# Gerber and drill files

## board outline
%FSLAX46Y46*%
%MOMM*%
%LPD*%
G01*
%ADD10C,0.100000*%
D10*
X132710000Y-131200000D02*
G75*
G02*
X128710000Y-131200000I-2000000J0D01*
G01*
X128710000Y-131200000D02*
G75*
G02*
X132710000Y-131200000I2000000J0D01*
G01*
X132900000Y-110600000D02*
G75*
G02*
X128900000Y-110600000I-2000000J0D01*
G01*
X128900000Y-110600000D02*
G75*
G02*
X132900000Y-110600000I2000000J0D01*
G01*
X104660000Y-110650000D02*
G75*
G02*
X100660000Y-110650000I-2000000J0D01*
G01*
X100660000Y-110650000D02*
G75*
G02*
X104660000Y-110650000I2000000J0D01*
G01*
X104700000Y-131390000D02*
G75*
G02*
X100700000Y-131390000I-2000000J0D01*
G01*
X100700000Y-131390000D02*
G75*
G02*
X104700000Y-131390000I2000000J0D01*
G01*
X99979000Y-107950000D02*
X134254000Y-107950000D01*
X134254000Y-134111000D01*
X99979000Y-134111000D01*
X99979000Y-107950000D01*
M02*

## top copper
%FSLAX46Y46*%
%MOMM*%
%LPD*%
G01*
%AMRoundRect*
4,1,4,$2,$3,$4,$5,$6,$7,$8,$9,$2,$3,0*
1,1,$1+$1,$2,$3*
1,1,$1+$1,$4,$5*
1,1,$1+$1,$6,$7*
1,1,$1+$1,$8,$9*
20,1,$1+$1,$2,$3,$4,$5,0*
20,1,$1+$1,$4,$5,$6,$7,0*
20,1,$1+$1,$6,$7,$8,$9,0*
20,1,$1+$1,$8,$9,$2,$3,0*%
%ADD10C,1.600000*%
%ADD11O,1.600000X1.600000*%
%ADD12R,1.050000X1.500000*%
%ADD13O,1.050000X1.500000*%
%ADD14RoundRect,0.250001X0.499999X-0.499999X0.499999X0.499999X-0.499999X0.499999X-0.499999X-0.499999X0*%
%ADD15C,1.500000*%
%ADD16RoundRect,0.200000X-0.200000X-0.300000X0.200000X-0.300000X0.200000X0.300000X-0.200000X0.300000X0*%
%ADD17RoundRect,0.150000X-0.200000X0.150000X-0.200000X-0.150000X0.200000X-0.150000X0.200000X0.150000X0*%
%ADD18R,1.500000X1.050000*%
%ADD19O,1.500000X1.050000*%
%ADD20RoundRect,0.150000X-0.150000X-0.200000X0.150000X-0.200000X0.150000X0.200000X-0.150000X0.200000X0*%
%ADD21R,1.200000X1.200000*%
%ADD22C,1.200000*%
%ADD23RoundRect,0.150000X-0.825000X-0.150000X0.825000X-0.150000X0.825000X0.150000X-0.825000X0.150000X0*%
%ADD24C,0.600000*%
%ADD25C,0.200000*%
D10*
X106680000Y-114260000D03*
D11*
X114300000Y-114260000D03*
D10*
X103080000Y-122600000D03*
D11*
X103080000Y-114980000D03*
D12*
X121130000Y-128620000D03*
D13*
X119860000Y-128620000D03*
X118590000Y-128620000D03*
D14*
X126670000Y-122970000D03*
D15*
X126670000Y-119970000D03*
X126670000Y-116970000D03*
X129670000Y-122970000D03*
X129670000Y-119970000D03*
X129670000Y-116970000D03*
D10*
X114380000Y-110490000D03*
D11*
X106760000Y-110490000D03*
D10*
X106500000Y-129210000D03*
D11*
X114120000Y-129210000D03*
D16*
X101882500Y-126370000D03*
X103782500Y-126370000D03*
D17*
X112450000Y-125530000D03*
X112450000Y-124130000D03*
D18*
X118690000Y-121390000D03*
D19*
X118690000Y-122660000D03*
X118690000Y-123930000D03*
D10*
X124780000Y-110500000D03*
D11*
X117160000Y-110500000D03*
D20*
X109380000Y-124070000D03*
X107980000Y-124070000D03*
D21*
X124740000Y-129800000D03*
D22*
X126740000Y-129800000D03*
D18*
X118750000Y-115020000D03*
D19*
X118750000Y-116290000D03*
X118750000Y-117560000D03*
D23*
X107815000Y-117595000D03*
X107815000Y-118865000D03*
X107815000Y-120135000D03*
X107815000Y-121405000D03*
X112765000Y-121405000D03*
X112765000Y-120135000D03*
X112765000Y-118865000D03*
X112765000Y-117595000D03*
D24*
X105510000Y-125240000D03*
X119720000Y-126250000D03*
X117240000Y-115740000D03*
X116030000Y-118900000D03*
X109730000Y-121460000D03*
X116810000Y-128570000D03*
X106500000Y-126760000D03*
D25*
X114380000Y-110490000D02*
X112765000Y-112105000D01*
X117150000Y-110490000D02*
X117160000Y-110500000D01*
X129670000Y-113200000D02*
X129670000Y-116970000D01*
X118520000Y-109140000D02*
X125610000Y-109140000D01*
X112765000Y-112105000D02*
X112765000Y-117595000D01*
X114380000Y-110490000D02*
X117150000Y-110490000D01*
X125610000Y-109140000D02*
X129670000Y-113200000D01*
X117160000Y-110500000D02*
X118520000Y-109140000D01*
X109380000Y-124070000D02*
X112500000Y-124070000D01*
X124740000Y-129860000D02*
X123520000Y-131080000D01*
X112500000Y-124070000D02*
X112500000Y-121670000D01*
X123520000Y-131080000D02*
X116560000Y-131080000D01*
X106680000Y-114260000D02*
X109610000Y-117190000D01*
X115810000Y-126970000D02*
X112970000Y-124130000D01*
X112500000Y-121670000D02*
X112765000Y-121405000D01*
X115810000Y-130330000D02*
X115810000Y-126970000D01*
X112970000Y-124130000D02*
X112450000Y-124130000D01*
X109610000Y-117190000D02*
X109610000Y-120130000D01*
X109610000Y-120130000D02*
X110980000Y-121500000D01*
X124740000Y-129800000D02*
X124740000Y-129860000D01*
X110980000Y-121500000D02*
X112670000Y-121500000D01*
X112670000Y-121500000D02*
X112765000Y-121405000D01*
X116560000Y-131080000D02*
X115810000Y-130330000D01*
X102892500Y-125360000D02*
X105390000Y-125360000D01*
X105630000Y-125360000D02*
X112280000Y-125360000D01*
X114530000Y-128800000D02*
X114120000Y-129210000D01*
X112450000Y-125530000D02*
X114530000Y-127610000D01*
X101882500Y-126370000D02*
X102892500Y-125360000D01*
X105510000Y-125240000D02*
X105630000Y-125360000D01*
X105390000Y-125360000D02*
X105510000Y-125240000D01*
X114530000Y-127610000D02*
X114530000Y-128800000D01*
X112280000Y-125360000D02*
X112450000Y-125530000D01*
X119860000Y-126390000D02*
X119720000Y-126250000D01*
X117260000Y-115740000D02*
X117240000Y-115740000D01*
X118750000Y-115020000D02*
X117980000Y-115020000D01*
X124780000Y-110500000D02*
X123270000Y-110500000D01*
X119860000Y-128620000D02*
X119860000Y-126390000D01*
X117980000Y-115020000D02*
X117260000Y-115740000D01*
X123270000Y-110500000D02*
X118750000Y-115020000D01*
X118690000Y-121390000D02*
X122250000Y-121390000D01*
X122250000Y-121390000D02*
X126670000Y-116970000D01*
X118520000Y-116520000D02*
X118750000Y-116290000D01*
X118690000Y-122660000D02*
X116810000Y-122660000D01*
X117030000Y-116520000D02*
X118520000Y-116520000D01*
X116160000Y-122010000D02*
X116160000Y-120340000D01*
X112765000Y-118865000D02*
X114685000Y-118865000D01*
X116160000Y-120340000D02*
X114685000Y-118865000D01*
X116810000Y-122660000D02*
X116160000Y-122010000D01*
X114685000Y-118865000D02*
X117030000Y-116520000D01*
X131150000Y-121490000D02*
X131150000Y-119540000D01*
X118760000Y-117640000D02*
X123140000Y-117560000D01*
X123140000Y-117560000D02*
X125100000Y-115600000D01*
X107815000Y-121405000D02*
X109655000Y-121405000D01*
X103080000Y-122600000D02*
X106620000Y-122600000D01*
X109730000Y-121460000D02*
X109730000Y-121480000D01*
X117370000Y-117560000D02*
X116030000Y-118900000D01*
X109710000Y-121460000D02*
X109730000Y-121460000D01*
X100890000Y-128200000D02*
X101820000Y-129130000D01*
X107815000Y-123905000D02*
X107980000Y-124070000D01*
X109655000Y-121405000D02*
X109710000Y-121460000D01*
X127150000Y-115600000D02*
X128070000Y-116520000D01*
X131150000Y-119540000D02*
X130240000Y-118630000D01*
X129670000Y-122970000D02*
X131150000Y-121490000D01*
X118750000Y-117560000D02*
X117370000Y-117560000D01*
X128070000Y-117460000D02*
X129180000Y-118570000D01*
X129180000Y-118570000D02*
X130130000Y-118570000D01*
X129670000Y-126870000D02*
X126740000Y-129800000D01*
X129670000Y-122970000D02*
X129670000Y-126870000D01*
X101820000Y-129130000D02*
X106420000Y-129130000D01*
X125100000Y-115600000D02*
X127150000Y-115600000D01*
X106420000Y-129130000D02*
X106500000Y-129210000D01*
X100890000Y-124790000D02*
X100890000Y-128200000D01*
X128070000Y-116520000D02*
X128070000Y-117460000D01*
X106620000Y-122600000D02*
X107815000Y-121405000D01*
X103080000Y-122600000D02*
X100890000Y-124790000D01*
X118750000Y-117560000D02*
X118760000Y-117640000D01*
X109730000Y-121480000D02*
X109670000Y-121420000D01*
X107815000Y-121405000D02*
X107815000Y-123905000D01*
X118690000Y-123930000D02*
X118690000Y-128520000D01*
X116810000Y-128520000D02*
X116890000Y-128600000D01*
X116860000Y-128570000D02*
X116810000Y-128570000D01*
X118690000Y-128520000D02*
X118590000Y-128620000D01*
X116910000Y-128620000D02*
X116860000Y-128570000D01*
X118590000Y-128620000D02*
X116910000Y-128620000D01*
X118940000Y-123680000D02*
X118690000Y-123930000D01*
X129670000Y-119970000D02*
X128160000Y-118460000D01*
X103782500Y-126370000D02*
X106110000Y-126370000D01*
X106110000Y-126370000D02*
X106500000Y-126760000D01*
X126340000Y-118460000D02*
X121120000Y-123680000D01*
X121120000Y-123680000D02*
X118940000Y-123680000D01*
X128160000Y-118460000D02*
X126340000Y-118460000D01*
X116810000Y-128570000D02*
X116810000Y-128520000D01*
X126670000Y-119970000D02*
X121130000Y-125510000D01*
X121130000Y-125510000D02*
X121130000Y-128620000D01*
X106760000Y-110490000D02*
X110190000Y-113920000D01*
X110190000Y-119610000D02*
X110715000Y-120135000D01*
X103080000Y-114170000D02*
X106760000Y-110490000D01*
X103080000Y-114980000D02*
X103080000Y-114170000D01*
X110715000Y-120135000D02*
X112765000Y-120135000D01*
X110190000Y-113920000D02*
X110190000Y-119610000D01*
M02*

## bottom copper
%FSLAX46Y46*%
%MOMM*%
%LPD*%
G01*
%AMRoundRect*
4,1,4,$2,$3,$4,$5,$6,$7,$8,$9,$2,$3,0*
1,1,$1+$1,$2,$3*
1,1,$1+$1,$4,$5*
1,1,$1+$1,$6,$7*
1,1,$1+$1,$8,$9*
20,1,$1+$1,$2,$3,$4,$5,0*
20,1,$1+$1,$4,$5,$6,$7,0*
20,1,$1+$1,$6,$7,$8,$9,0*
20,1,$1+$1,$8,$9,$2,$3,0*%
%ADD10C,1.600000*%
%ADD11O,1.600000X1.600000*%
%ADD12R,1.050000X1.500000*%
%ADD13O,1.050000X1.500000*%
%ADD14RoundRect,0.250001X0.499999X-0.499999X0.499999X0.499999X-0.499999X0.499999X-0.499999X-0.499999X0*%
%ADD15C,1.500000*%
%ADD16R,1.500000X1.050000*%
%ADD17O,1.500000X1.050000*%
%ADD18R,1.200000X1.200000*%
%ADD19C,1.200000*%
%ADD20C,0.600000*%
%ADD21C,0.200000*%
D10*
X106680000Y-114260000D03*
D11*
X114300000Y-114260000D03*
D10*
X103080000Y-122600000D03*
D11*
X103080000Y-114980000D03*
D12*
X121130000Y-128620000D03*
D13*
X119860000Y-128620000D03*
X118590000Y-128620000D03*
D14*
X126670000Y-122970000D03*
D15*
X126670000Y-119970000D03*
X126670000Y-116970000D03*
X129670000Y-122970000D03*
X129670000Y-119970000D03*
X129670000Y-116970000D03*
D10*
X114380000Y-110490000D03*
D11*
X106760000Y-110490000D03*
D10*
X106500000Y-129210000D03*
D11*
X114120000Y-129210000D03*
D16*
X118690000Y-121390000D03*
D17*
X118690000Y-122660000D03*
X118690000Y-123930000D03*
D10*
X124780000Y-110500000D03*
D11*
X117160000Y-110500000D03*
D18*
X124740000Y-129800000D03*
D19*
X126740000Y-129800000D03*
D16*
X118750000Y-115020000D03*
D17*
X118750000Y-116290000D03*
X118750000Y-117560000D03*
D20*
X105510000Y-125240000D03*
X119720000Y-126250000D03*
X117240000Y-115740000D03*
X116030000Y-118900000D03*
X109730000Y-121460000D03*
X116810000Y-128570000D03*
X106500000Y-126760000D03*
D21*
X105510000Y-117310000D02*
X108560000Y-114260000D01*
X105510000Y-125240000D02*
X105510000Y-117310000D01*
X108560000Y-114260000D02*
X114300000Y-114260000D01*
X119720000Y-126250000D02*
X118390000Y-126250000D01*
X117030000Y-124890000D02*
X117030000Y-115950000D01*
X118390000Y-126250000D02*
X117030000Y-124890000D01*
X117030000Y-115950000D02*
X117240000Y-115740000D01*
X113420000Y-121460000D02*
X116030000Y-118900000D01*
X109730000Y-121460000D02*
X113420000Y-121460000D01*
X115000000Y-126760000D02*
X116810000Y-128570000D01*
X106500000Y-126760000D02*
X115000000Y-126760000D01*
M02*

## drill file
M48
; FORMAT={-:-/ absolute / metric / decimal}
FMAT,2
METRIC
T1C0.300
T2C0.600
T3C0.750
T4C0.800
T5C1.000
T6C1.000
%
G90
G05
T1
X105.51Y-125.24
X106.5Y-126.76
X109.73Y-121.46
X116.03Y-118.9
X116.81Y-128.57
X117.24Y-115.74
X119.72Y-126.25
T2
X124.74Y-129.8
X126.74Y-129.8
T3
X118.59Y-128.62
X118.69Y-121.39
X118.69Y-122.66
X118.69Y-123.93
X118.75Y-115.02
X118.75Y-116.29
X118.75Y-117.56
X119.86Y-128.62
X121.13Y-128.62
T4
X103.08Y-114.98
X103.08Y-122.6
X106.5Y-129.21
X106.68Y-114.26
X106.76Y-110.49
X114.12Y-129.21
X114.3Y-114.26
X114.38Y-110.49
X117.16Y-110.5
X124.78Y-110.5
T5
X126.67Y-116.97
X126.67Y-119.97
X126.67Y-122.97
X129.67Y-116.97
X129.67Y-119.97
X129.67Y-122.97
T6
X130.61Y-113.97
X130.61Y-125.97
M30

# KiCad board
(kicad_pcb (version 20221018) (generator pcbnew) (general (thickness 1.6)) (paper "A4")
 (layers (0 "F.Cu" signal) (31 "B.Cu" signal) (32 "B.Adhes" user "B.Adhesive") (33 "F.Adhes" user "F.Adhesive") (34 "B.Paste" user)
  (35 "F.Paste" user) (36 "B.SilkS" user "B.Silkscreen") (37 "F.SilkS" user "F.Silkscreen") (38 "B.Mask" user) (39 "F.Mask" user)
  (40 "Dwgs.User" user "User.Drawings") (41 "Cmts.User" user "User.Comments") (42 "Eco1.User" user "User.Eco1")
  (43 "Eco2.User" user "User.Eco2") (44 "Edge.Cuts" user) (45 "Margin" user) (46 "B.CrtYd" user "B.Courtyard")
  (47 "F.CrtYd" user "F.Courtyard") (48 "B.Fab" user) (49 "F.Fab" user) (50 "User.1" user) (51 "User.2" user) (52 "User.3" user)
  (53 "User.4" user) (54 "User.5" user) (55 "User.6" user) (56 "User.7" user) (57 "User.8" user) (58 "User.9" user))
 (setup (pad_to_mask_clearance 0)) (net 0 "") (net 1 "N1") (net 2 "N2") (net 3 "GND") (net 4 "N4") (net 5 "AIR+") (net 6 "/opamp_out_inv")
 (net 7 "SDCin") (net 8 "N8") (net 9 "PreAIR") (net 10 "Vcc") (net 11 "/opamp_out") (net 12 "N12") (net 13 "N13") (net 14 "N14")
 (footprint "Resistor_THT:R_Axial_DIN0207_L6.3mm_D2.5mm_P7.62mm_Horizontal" (layer "F.Cu") (at 106.68 114.26)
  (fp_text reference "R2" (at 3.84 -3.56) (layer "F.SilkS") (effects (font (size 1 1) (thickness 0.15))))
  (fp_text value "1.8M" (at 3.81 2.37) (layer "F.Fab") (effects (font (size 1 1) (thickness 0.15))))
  (pad "1" thru_hole circle (at 0 0) (size 1.6 1.6) (drill 0.8) (layers "*.Cu" "*.Mask") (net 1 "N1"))
  (pad "2" thru_hole oval (at 7.62 0) (size 1.6 1.6) (drill 0.8) (layers "*.Cu" "*.Mask") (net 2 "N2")))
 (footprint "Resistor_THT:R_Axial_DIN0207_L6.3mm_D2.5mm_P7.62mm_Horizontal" (layer "F.Cu") (at 103.08 122.6 90)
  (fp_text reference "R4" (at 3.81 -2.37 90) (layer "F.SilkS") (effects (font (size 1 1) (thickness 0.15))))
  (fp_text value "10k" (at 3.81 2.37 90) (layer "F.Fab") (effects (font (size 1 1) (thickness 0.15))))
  (pad "1" thru_hole circle (at 0 0 90) (size 1.6 1.6) (drill 0.8) (layers "*.Cu" "*.Mask") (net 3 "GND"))
  (pad "2" thru_hole oval (at 7.62 0 90) (size 1.6 1.6) (drill 0.8) (layers "*.Cu" "*.Mask") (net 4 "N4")))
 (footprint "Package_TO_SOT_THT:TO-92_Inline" (layer "F.Cu") (at 121.13 128.62 180)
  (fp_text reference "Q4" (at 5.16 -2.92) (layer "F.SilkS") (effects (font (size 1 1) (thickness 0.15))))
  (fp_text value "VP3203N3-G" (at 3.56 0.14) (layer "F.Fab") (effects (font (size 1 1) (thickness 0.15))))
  (pad "1" thru_hole rect (at 0 0 180) (size 1.05 1.5) (drill 0.75) (layers "*.Cu" "*.Mask") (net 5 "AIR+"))
  (pad "2" thru_hole oval (at 1.27 0 180) (size 1.05 1.5) (drill 0.75) (layers "*.Cu" "*.Mask") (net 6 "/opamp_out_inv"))
  (pad "3" thru_hole oval (at 2.54 0 180) (size 1.05 1.5) (drill 0.75) (layers "*.Cu" "*.Mask") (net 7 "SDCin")))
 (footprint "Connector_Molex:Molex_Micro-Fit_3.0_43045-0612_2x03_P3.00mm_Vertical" (layer "F.Cu") (at 126.67 122.97 90)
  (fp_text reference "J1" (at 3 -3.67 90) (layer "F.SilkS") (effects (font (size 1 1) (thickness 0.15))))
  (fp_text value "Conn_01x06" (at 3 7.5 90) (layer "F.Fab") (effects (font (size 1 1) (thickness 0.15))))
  (pad "" np_thru_hole circle (at -3 3.94 90) (size 1 1) (drill 1) (layers "*.Cu" "*.Mask"))
  (pad "" np_thru_hole circle (at 9 3.94 90) (size 1 1) (drill 1) (layers "*.Cu" "*.Mask"))
  (pad "1" thru_hole roundrect (at 0 0 90) (size 1.5 1.5) (drill 1) (layers "*.Cu" "*.Mask") (roundrect_rratio 0.166667) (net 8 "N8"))
  (pad "2" thru_hole circle (at 3 0 90) (size 1.5 1.5) (drill 1) (layers "*.Cu" "*.Mask") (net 5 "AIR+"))
  (pad "3" thru_hole circle (at 6 0 90) (size 1.5 1.5) (drill 1) (layers "*.Cu" "*.Mask") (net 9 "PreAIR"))
  (pad "4" thru_hole circle (at 0 3 90) (size 1.5 1.5) (drill 1) (layers "*.Cu" "*.Mask") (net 3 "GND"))
  (pad "5" thru_hole circle (at 3 3 90) (size 1.5 1.5) (drill 1) (layers "*.Cu" "*.Mask") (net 7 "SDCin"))
  (pad "6" thru_hole circle (at 6 3 90) (size 1.5 1.5) (drill 1) (layers "*.Cu" "*.Mask") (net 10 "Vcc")))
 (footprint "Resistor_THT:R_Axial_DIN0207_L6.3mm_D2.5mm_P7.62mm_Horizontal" (layer "F.Cu") (at 114.38 110.49 180)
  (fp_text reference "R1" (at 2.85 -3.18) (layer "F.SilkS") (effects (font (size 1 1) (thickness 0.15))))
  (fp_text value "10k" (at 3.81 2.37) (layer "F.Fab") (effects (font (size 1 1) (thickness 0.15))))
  (pad "1" thru_hole circle (at 0 0 180) (size 1.6 1.6) (drill 0.8) (layers "*.Cu" "*.Mask") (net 10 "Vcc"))
  (pad "2" thru_hole oval (at 7.62 0 180) (size 1.6 1.6) (drill 0.8) (layers "*.Cu" "*.Mask") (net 4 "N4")))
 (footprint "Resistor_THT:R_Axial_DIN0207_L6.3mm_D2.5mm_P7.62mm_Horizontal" (layer "F.Cu") (at 106.5 129.21)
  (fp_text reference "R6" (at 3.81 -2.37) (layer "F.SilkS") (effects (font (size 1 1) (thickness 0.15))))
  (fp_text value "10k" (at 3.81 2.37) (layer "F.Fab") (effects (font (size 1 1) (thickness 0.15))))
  (pad "1" thru_hole circle (at 0 0) (size 1.6 1.6) (drill 0.8) (layers "*.Cu" "*.Mask") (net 3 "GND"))
  (pad "2" thru_hole oval (at 7.62 0) (size 1.6 1.6) (drill 0.8) (layers "*.Cu" "*.Mask") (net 2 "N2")))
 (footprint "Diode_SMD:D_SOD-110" (layer "F.Cu") (at 102.8325 126.37)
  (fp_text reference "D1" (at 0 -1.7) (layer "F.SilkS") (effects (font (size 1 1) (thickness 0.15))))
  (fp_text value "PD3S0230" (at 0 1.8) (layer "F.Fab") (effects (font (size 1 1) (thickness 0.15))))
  (pad "1" smd roundrect (at -0.95 0) (size 0.8 1) (layers "F.Cu" "F.Paste" "F.Mask") (roundrect_rratio 0.25) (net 2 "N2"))
  (pad "2" smd roundrect (at 0.95 0) (size 0.8 1) (layers "F.Cu" "F.Paste" "F.Mask") (roundrect_rratio 0.25) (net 7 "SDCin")))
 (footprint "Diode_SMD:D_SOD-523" (layer "F.Cu") (at 112.45 124.83 90)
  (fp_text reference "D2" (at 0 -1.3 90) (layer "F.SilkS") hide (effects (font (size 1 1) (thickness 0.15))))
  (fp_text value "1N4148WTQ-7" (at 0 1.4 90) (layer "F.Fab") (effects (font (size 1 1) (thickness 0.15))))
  (pad "1" smd roundrect (at -0.7 0 270) (size 0.6 0.7) (layers "F.Cu" "F.Paste" "F.Mask") (roundrect_rratio 0.25) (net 2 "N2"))
  (pad "2" smd roundrect (at 0.7 0 270) (size 0.6 0.7) (layers "F.Cu" "F.Paste" "F.Mask") (roundrect_rratio 0.25) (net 1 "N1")))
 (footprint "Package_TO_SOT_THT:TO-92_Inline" (layer "F.Cu") (at 118.69 121.39 -90)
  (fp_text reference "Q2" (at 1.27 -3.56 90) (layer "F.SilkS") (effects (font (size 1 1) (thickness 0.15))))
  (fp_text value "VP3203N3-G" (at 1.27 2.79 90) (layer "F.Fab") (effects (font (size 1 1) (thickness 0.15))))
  (pad "1" thru_hole rect (at 0 0 270) (size 1.05 1.5) (drill 0.75) (layers "*.Cu" "*.Mask") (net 9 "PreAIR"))
  (pad "2" thru_hole oval (at 1.27 0 270) (size 1.05 1.5) (drill 0.75) (layers "*.Cu" "*.Mask") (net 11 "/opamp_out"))
  (pad "3" thru_hole oval (at 2.54 0 270) (size 1.05 1.5) (drill 0.75) (layers "*.Cu" "*.Mask") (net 7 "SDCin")))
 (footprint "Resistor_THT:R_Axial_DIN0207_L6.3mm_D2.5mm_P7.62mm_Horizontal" (layer "F.Cu") (at 124.78 110.5 180)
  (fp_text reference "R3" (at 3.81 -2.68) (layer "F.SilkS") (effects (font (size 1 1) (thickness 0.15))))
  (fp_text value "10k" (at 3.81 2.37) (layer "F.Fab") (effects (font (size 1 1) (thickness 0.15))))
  (pad "1" thru_hole circle (at 0 0 180) (size 1.6 1.6) (drill 0.8) (layers "*.Cu" "*.Mask") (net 6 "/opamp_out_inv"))
  (pad "2" thru_hole oval (at 7.62 0 180) (size 1.6 1.6) (drill 0.8) (layers "*.Cu" "*.Mask") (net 10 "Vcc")))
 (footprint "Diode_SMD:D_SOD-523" (layer "F.Cu") (at 108.68 124.07 180)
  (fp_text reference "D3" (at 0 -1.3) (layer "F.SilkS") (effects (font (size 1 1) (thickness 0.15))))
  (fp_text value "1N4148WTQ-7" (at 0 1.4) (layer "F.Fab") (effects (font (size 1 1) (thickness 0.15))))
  (pad "1" smd roundrect (at -0.7 0) (size 0.6 0.7) (layers "F.Cu" "F.Paste" "F.Mask") (roundrect_rratio 0.25) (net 1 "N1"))
  (pad "2" smd roundrect (at 0.7 0) (size 0.6 0.7) (layers "F.Cu" "F.Paste" "F.Mask") (roundrect_rratio 0.25) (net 3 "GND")))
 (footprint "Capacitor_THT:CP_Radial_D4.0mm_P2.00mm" (layer "F.Cu") (at 124.74 129.8)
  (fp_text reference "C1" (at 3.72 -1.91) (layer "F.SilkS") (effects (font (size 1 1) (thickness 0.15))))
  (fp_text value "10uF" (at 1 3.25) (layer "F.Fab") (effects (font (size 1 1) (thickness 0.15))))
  (pad "1" thru_hole rect (at 0 0) (size 1.2 1.2) (drill 0.6) (layers "*.Cu" "*.Mask") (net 1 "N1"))
  (pad "2" thru_hole circle (at 2 0) (size 1.2 1.2) (drill 0.6) (layers "*.Cu" "*.Mask") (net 3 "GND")))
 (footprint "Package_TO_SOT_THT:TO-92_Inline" (layer "F.Cu") (at 118.75 115.02 -90)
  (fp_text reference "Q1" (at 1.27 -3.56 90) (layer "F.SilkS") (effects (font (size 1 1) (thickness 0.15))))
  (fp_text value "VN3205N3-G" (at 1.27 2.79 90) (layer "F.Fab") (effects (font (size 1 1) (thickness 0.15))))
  (pad "1" thru_hole rect (at 0 0 270) (size 1.05 1.5) (drill 0.75) (layers "*.Cu" "*.Mask") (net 6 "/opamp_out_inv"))
  (pad "2" thru_hole oval (at 1.27 0 270) (size 1.05 1.5) (drill 0.75) (layers "*.Cu" "*.Mask") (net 11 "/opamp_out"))
  (pad "3" thru_hole oval (at 2.54 0 270) (size 1.05 1.5) (drill 0.75) (layers "*.Cu" "*.Mask") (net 3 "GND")))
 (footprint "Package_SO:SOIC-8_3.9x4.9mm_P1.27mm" (layer "F.Cu") (at 110.29 119.5)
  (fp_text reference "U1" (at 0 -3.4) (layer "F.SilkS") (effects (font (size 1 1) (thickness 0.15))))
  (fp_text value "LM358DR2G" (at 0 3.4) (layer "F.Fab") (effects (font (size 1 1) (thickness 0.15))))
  (pad "1" smd roundrect (at -2.475 -1.905) (size 1.95 0.6) (layers "F.Cu" "F.Paste" "F.Mask") (roundrect_rratio 0.25) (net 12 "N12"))
  (pad "2" smd roundrect (at -2.475 -0.635) (size 1.95 0.6) (layers "F.Cu" "F.Paste" "F.Mask") (roundrect_rratio 0.25) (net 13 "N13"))
  (pad "3" smd roundrect (at -2.475 0.635) (size 1.95 0.6) (layers "F.Cu" "F.Paste" "F.Mask") (roundrect_rratio 0.25) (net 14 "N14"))
  (pad "4" smd roundrect (at -2.475 1.905) (size 1.95 0.6) (layers "F.Cu" "F.Paste" "F.Mask") (roundrect_rratio 0.25) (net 3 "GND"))
  (pad "5" smd roundrect (at 2.475 1.905) (size 1.95 0.6) (layers "F.Cu" "F.Paste" "F.Mask") (roundrect_rratio 0.25) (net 1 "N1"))
  (pad "6" smd roundrect (at 2.475 0.635) (size 1.95 0.6) (layers "F.Cu" "F.Paste" "F.Mask") (roundrect_rratio 0.25) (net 4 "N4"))
  (pad "7" smd roundrect (at 2.475 -0.635) (size 1.95 0.6) (layers "F.Cu" "F.Paste" "F.Mask") (roundrect_rratio 0.25) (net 11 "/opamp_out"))
  (pad "8" smd roundrect (at 2.475 -1.905) (size 1.95 0.6) (layers "F.Cu" "F.Paste" "F.Mask") (roundrect_rratio 0.25) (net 10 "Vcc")))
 (gr_circle (center 130.71 131.2) (end 132.71 131.2) (stroke (width 0.1) (type default)) (fill none) (layer "Edge.Cuts"))
 (gr_circle (center 130.9 110.6) (end 132.9 110.6) (stroke (width 0.1) (type default)) (fill none) (layer "Edge.Cuts"))
 (gr_circle (center 102.66 110.65) (end 104.66 110.65) (stroke (width 0.1) (type default)) (fill none) (layer "Edge.Cuts"))
 (gr_circle (center 102.7 131.39) (end 104.7 131.39) (stroke (width 0.1) (type default)) (fill none) (layer "Edge.Cuts"))
 (gr_rect (start 99.979 107.95) (end 134.254 134.111) (stroke (width 0.1) (type solid)) (fill none) (layer "Edge.Cuts"))
 (segment (start 114.38 110.49) (end 112.765 112.105) (width 0.2) (layer "F.Cu") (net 10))
 (segment (start 117.15 110.49) (end 117.16 110.5) (width 0.2) (layer "F.Cu") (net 10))
 (segment (start 129.67 113.2) (end 129.67 116.97) (width 0.2) (layer "F.Cu") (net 10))
 (segment (start 118.52 109.14) (end 125.61 109.14) (width 0.2) (layer "F.Cu") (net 10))
 (segment (start 112.765 112.105) (end 112.765 117.595) (width 0.2) (layer "F.Cu") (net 10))
 (segment (start 114.38 110.49) (end 117.15 110.49) (width 0.2) (layer "F.Cu") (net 10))
 (segment (start 125.61 109.14) (end 129.67 113.2) (width 0.2) (layer "F.Cu") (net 10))
 (segment (start 117.16 110.5) (end 118.52 109.14) (width 0.2) (layer "F.Cu") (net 10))
 (segment (start 109.38 124.07) (end 112.5 124.07) (width 0.2) (layer "F.Cu") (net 1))
 (segment (start 124.74 129.86) (end 123.52 131.08) (width 0.2) (layer "F.Cu") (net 1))
 (segment (start 112.5 124.07) (end 112.5 121.67) (width 0.2) (layer "F.Cu") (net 1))
 (segment (start 123.52 131.08) (end 116.56 131.08) (width 0.2) (layer "F.Cu") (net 1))
 (segment (start 106.68 114.26) (end 109.61 117.19) (width 0.2) (layer "F.Cu") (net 1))
 (segment (start 115.81 126.97) (end 112.97 124.13) (width 0.2) (layer "F.Cu") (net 1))
 (segment (start 112.5 121.67) (end 112.765 121.405) (width 0.2) (layer "F.Cu") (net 1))
 (segment (start 115.81 130.33) (end 115.81 126.97) (width 0.2) (layer "F.Cu") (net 1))
 (segment (start 112.97 124.13) (end 112.45 124.13) (width 0.2) (layer "F.Cu") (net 1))
 (segment (start 109.61 117.19) (end 109.61 120.13) (width 0.2) (layer "F.Cu") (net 1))
 (segment (start 109.61 120.13) (end 110.98 121.5) (width 0.2) (layer "F.Cu") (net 1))
 (segment (start 124.74 129.8) (end 124.74 129.86) (width 0.2) (layer "F.Cu") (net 1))
 (segment (start 110.98 121.5) (end 112.67 121.5) (width 0.2) (layer "F.Cu") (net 1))
 (segment (start 112.67 121.5) (end 112.765 121.405) (width 0.2) (layer "F.Cu") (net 1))
 (segment (start 116.56 131.08) (end 115.81 130.33) (width 0.2) (layer "F.Cu") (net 1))
 (segment (start 102.8925 125.36) (end 105.39 125.36) (width 0.2) (layer "F.Cu") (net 2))
 (segment (start 105.63 125.36) (end 112.28 125.36) (width 0.2) (layer "F.Cu") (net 2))
 (segment (start 114.53 128.8) (end 114.12 129.21) (width 0.2) (layer "F.Cu") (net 2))
 (segment (start 112.45 125.53) (end 114.53 127.61) (width 0.2) (layer "F.Cu") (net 2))
 (segment (start 101.8825 126.37) (end 102.8925 125.36) (width 0.2) (layer "F.Cu") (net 2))
 (segment (start 105.51 125.24) (end 105.63 125.36) (width 0.2) (layer "F.Cu") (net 2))
 (segment (start 105.39 125.36) (end 105.51 125.24) (width 0.2) (layer "F.Cu") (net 2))
 (segment (start 114.53 127.61) (end 114.53 128.8) (width 0.2) (layer "F.Cu") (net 2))
 (segment (start 112.28 125.36) (end 112.45 125.53) (width 0.2) (layer "F.Cu") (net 2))
 (via (at 105.51 125.24) (size 0.6) (drill 0.3) (layers "F.Cu" "B.Cu") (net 2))
 (segment (start 105.51 117.31) (end 108.56 114.26) (width 0.2) (layer "B.Cu") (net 2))
 (segment (start 105.51 125.24) (end 105.51 117.31) (width 0.2) (layer "B.Cu") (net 2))
 (segment (start 108.56 114.26) (end 114.3 114.26) (width 0.2) (layer "B.Cu") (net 2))
 (segment (start 119.86 126.39) (end 119.72 126.25) (width 0.2) (layer "F.Cu") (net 6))
 (segment (start 117.26 115.74) (end 117.24 115.74) (width 0.2) (layer "F.Cu") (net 6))
 (segment (start 118.75 115.02) (end 117.98 115.02) (width 0.2) (layer "F.Cu") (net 6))
 (segment (start 124.78 110.5) (end 123.27 110.5) (width 0.2) (layer "F.Cu") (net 6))
 (segment (start 119.86 128.62) (end 119.86 126.39) (width 0.2) (layer "F.Cu") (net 6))
 (segment (start 117.98 115.02) (end 117.26 115.74) (width 0.2) (layer "F.Cu") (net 6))
 (segment (start 123.27 110.5) (end 118.75 115.02) (width 0.2) (layer "F.Cu") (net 6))
 (via (at 119.72 126.25) (size 0.6) (drill 0.3) (layers "F.Cu" "B.Cu") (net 6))
 (via (at 117.24 115.74) (size 0.6) (drill 0.3) (layers "F.Cu" "B.Cu") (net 6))
 (segment (start 119.72 126.25) (end 118.39 126.25) (width 0.2) (layer "B.Cu") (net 6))
 (segment (start 117.03 124.89) (end 117.03 115.95) (width 0.2) (layer "B.Cu") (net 6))
 (segment (start 118.39 126.25) (end 117.03 124.89) (width 0.2) (layer "B.Cu") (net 6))
 (segment (start 117.03 115.95) (end 117.24 115.74) (width 0.2) (layer "B.Cu") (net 6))
 (segment (start 118.69 121.39) (end 122.25 121.39) (width 0.2) (layer "F.Cu") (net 9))
 (segment (start 122.25 121.39) (end 126.67 116.97) (width 0.2) (layer "F.Cu") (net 9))
 (segment (start 118.52 116.52) (end 118.75 116.29) (width 0.2) (layer "F.Cu") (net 11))
 (segment (start 118.69 122.66) (end 116.81 122.66) (width 0.2) (layer "F.Cu") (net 11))
 (segment (start 117.03 116.52) (end 118.52 116.52) (width 0.2) (layer "F.Cu") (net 11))
 (segment (start 116.16 122.01) (end 116.16 120.34) (width 0.2) (layer "F.Cu") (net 11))
 (segment (start 112.765 118.865) (end 114.685 118.865) (width 0.2) (layer "F.Cu") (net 11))
 (segment (start 116.16 120.34) (end 114.685 118.865) (width 0.2) (layer "F.Cu") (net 11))
 (segment (start 116.81 122.66) (end 116.16 122.01) (width 0.2) (layer "F.Cu") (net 11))
 (segment (start 114.685 118.865) (end 117.03 116.52) (width 0.2) (layer "F.Cu") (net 11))
 (segment (start 131.15 121.49) (end 131.15 119.54) (width 0.2) (layer "F.Cu") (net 3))
 (segment (start 118.76 117.64) (end 123.14 117.56) (width 0.2) (layer "F.Cu") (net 3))
 (segment (start 123.14 117.56) (end 125.1 115.6) (width 0.2) (layer "F.Cu") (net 3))
 (segment (start 107.815 121.405) (end 109.655 121.405) (width 0.2) (layer "F.Cu") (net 3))
 (segment (start 103.08 122.6) (end 106.62 122.6) (width 0.2) (layer "F.Cu") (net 3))
 (segment (start 109.73 121.46) (end 109.73 121.48) (width 0.2) (layer "F.Cu") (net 3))
 (segment (start 117.37 117.56) (end 116.03 118.9) (width 0.2) (layer "F.Cu") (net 3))
 (segment (start 109.71 121.46) (end 109.73 121.46) (width 0.2) (layer "F.Cu") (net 3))
 (segment (start 100.89 128.2) (end 101.82 129.13) (width 0.2) (layer "F.Cu") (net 3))
 (segment (start 107.815 123.905) (end 107.98 124.07) (width 0.2) (layer "F.Cu") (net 3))
 (segment (start 109.655 121.405) (end 109.71 121.46) (width 0.2) (layer "F.Cu") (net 3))
 (segment (start 127.15 115.6) (end 128.07 116.52) (width 0.2) (layer "F.Cu") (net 3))
 (segment (start 131.15 119.54) (end 130.24 118.63) (width 0.2) (layer "F.Cu") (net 3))
 (segment (start 129.67 122.97) (end 131.15 121.49) (width 0.2) (layer "F.Cu") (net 3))
 (segment (start 118.75 117.56) (end 117.37 117.56) (width 0.2) (layer "F.Cu") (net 3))
 (segment (start 128.07 117.46) (end 129.18 118.57) (width 0.2) (layer "F.Cu") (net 3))
 (segment (start 129.18 118.57) (end 130.13 118.57) (width 0.2) (layer "F.Cu") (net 3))
 (segment (start 129.67 126.87) (end 126.74 129.8) (width 0.2) (layer "F.Cu") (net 3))
 (segment (start 129.67 122.97) (end 129.67 126.87) (width 0.2) (layer "F.Cu") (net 3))
 (segment (start 101.82 129.13) (end 106.42 129.13) (width 0.2) (layer "F.Cu") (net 3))
 (segment (start 125.1 115.6) (end 127.15 115.6) (width 0.2) (layer "F.Cu") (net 3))
 (segment (start 106.42 129.13) (end 106.5 129.21) (width 0.2) (layer "F.Cu") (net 3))
 (segment (start 100.89 124.79) (end 100.89 128.2) (width 0.2) (layer "F.Cu") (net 3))
 (segment (start 128.07 116.52) (end 128.07 117.46) (width 0.2) (layer "F.Cu") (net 3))
 (segment (start 106.62 122.6) (end 107.815 121.405) (width 0.2) (layer "F.Cu") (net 3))
 (segment (start 103.08 122.6) (end 100.89 124.79) (width 0.2) (layer "F.Cu") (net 3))
 (segment (start 118.75 117.56) (end 118.76 117.64) (width 0.2) (layer "F.Cu") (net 3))
 (segment (start 109.73 121.48) (end 109.67 121.42) (width 0.2) (layer "F.Cu") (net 3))
 (segment (start 107.815 121.405) (end 107.815 123.905) (width 0.2) (layer "F.Cu") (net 3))
 (via (at 116.03 118.9) (size 0.6) (drill 0.3) (layers "F.Cu" "B.Cu") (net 3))
 (via (at 109.73 121.46) (size 0.6) (drill 0.3) (layers "F.Cu" "B.Cu") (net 3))
 (segment (start 113.42 121.46) (end 116.03 118.9) (width 0.2) (layer "B.Cu") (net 3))
 (segment (start 109.73 121.46) (end 113.42 121.46) (width 0.2) (layer "B.Cu") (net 3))
 (segment (start 118.69 123.93) (end 118.69 128.52) (width 0.2) (layer "F.Cu") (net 7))
 (segment (start 116.81 128.52) (end 116.89 128.6) (width 0.2) (layer "F.Cu") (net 7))
 (segment (start 116.86 128.57) (end 116.81 128.57) (width 0.2) (layer "F.Cu") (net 7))
 (segment (start 118.69 128.52) (end 118.59 128.62) (width 0.2) (layer "F.Cu") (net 7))
 (segment (start 116.91 128.62) (end 116.86 128.57) (width 0.2) (layer "F.Cu") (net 7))
 (segment (start 118.59 128.62) (end 116.91 128.62) (width 0.2) (layer "F.Cu") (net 7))
 (segment (start 118.94 123.68) (end 118.69 123.93) (width 0.2) (layer "F.Cu") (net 7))
 (segment (start 129.67 119.97) (end 128.16 118.46) (width 0.2) (layer "F.Cu") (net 7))
 (segment (start 103.7825 126.37) (end 106.11 126.37) (width 0.2) (layer "F.Cu") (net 7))
 (segment (start 106.11 126.37) (end 106.5 126.76) (width 0.2) (layer "F.Cu") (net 7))
 (segment (start 126.34 118.46) (end 121.12 123.68) (width 0.2) (layer "F.Cu") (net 7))
 (segment (start 121.12 123.68) (end 118.94 123.68) (width 0.2) (layer "F.Cu") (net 7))
 (segment (start 128.16 118.46) (end 126.34 118.46) (width 0.2) (layer "F.Cu") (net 7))
 (segment (start 116.81 128.57) (end 116.81 128.52) (width 0.2) (layer "F.Cu") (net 7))
 (via (at 116.81 128.57) (size 0.6) (drill 0.3) (layers "F.Cu" "B.Cu") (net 7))
 (via (at 106.5 126.76) (size 0.6) (drill 0.3) (layers "F.Cu" "B.Cu") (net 7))
 (segment (start 115 126.76) (end 116.81 128.57) (width 0.2) (layer "B.Cu") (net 7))
 (segment (start 106.5 126.76) (end 115 126.76) (width 0.2) (layer "B.Cu") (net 7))
 (segment (start 126.67 119.97) (end 121.13 125.51) (width 0.2) (layer "F.Cu") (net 5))
 (segment (start 121.13 125.51) (end 121.13 128.62) (width 0.2) (layer "F.Cu") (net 5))
 (segment (start 106.76 110.49) (end 110.19 113.92) (width 0.2) (layer "F.Cu") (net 4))
 (segment (start 110.19 119.61) (end 110.715 120.135) (width 0.2) (layer "F.Cu") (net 4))
 (segment (start 103.08 114.17) (end 106.76 110.49) (width 0.2) (layer "F.Cu") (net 4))
 (segment (start 103.08 114.98) (end 103.08 114.17) (width 0.2) (layer "F.Cu") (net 4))
 (segment (start 110.715 120.135) (end 112.765 120.135) (width 0.2) (layer "F.Cu") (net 4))
 (segment (start 110.19 113.92) (end 110.19 119.61) (width 0.2) (layer "F.Cu") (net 4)))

